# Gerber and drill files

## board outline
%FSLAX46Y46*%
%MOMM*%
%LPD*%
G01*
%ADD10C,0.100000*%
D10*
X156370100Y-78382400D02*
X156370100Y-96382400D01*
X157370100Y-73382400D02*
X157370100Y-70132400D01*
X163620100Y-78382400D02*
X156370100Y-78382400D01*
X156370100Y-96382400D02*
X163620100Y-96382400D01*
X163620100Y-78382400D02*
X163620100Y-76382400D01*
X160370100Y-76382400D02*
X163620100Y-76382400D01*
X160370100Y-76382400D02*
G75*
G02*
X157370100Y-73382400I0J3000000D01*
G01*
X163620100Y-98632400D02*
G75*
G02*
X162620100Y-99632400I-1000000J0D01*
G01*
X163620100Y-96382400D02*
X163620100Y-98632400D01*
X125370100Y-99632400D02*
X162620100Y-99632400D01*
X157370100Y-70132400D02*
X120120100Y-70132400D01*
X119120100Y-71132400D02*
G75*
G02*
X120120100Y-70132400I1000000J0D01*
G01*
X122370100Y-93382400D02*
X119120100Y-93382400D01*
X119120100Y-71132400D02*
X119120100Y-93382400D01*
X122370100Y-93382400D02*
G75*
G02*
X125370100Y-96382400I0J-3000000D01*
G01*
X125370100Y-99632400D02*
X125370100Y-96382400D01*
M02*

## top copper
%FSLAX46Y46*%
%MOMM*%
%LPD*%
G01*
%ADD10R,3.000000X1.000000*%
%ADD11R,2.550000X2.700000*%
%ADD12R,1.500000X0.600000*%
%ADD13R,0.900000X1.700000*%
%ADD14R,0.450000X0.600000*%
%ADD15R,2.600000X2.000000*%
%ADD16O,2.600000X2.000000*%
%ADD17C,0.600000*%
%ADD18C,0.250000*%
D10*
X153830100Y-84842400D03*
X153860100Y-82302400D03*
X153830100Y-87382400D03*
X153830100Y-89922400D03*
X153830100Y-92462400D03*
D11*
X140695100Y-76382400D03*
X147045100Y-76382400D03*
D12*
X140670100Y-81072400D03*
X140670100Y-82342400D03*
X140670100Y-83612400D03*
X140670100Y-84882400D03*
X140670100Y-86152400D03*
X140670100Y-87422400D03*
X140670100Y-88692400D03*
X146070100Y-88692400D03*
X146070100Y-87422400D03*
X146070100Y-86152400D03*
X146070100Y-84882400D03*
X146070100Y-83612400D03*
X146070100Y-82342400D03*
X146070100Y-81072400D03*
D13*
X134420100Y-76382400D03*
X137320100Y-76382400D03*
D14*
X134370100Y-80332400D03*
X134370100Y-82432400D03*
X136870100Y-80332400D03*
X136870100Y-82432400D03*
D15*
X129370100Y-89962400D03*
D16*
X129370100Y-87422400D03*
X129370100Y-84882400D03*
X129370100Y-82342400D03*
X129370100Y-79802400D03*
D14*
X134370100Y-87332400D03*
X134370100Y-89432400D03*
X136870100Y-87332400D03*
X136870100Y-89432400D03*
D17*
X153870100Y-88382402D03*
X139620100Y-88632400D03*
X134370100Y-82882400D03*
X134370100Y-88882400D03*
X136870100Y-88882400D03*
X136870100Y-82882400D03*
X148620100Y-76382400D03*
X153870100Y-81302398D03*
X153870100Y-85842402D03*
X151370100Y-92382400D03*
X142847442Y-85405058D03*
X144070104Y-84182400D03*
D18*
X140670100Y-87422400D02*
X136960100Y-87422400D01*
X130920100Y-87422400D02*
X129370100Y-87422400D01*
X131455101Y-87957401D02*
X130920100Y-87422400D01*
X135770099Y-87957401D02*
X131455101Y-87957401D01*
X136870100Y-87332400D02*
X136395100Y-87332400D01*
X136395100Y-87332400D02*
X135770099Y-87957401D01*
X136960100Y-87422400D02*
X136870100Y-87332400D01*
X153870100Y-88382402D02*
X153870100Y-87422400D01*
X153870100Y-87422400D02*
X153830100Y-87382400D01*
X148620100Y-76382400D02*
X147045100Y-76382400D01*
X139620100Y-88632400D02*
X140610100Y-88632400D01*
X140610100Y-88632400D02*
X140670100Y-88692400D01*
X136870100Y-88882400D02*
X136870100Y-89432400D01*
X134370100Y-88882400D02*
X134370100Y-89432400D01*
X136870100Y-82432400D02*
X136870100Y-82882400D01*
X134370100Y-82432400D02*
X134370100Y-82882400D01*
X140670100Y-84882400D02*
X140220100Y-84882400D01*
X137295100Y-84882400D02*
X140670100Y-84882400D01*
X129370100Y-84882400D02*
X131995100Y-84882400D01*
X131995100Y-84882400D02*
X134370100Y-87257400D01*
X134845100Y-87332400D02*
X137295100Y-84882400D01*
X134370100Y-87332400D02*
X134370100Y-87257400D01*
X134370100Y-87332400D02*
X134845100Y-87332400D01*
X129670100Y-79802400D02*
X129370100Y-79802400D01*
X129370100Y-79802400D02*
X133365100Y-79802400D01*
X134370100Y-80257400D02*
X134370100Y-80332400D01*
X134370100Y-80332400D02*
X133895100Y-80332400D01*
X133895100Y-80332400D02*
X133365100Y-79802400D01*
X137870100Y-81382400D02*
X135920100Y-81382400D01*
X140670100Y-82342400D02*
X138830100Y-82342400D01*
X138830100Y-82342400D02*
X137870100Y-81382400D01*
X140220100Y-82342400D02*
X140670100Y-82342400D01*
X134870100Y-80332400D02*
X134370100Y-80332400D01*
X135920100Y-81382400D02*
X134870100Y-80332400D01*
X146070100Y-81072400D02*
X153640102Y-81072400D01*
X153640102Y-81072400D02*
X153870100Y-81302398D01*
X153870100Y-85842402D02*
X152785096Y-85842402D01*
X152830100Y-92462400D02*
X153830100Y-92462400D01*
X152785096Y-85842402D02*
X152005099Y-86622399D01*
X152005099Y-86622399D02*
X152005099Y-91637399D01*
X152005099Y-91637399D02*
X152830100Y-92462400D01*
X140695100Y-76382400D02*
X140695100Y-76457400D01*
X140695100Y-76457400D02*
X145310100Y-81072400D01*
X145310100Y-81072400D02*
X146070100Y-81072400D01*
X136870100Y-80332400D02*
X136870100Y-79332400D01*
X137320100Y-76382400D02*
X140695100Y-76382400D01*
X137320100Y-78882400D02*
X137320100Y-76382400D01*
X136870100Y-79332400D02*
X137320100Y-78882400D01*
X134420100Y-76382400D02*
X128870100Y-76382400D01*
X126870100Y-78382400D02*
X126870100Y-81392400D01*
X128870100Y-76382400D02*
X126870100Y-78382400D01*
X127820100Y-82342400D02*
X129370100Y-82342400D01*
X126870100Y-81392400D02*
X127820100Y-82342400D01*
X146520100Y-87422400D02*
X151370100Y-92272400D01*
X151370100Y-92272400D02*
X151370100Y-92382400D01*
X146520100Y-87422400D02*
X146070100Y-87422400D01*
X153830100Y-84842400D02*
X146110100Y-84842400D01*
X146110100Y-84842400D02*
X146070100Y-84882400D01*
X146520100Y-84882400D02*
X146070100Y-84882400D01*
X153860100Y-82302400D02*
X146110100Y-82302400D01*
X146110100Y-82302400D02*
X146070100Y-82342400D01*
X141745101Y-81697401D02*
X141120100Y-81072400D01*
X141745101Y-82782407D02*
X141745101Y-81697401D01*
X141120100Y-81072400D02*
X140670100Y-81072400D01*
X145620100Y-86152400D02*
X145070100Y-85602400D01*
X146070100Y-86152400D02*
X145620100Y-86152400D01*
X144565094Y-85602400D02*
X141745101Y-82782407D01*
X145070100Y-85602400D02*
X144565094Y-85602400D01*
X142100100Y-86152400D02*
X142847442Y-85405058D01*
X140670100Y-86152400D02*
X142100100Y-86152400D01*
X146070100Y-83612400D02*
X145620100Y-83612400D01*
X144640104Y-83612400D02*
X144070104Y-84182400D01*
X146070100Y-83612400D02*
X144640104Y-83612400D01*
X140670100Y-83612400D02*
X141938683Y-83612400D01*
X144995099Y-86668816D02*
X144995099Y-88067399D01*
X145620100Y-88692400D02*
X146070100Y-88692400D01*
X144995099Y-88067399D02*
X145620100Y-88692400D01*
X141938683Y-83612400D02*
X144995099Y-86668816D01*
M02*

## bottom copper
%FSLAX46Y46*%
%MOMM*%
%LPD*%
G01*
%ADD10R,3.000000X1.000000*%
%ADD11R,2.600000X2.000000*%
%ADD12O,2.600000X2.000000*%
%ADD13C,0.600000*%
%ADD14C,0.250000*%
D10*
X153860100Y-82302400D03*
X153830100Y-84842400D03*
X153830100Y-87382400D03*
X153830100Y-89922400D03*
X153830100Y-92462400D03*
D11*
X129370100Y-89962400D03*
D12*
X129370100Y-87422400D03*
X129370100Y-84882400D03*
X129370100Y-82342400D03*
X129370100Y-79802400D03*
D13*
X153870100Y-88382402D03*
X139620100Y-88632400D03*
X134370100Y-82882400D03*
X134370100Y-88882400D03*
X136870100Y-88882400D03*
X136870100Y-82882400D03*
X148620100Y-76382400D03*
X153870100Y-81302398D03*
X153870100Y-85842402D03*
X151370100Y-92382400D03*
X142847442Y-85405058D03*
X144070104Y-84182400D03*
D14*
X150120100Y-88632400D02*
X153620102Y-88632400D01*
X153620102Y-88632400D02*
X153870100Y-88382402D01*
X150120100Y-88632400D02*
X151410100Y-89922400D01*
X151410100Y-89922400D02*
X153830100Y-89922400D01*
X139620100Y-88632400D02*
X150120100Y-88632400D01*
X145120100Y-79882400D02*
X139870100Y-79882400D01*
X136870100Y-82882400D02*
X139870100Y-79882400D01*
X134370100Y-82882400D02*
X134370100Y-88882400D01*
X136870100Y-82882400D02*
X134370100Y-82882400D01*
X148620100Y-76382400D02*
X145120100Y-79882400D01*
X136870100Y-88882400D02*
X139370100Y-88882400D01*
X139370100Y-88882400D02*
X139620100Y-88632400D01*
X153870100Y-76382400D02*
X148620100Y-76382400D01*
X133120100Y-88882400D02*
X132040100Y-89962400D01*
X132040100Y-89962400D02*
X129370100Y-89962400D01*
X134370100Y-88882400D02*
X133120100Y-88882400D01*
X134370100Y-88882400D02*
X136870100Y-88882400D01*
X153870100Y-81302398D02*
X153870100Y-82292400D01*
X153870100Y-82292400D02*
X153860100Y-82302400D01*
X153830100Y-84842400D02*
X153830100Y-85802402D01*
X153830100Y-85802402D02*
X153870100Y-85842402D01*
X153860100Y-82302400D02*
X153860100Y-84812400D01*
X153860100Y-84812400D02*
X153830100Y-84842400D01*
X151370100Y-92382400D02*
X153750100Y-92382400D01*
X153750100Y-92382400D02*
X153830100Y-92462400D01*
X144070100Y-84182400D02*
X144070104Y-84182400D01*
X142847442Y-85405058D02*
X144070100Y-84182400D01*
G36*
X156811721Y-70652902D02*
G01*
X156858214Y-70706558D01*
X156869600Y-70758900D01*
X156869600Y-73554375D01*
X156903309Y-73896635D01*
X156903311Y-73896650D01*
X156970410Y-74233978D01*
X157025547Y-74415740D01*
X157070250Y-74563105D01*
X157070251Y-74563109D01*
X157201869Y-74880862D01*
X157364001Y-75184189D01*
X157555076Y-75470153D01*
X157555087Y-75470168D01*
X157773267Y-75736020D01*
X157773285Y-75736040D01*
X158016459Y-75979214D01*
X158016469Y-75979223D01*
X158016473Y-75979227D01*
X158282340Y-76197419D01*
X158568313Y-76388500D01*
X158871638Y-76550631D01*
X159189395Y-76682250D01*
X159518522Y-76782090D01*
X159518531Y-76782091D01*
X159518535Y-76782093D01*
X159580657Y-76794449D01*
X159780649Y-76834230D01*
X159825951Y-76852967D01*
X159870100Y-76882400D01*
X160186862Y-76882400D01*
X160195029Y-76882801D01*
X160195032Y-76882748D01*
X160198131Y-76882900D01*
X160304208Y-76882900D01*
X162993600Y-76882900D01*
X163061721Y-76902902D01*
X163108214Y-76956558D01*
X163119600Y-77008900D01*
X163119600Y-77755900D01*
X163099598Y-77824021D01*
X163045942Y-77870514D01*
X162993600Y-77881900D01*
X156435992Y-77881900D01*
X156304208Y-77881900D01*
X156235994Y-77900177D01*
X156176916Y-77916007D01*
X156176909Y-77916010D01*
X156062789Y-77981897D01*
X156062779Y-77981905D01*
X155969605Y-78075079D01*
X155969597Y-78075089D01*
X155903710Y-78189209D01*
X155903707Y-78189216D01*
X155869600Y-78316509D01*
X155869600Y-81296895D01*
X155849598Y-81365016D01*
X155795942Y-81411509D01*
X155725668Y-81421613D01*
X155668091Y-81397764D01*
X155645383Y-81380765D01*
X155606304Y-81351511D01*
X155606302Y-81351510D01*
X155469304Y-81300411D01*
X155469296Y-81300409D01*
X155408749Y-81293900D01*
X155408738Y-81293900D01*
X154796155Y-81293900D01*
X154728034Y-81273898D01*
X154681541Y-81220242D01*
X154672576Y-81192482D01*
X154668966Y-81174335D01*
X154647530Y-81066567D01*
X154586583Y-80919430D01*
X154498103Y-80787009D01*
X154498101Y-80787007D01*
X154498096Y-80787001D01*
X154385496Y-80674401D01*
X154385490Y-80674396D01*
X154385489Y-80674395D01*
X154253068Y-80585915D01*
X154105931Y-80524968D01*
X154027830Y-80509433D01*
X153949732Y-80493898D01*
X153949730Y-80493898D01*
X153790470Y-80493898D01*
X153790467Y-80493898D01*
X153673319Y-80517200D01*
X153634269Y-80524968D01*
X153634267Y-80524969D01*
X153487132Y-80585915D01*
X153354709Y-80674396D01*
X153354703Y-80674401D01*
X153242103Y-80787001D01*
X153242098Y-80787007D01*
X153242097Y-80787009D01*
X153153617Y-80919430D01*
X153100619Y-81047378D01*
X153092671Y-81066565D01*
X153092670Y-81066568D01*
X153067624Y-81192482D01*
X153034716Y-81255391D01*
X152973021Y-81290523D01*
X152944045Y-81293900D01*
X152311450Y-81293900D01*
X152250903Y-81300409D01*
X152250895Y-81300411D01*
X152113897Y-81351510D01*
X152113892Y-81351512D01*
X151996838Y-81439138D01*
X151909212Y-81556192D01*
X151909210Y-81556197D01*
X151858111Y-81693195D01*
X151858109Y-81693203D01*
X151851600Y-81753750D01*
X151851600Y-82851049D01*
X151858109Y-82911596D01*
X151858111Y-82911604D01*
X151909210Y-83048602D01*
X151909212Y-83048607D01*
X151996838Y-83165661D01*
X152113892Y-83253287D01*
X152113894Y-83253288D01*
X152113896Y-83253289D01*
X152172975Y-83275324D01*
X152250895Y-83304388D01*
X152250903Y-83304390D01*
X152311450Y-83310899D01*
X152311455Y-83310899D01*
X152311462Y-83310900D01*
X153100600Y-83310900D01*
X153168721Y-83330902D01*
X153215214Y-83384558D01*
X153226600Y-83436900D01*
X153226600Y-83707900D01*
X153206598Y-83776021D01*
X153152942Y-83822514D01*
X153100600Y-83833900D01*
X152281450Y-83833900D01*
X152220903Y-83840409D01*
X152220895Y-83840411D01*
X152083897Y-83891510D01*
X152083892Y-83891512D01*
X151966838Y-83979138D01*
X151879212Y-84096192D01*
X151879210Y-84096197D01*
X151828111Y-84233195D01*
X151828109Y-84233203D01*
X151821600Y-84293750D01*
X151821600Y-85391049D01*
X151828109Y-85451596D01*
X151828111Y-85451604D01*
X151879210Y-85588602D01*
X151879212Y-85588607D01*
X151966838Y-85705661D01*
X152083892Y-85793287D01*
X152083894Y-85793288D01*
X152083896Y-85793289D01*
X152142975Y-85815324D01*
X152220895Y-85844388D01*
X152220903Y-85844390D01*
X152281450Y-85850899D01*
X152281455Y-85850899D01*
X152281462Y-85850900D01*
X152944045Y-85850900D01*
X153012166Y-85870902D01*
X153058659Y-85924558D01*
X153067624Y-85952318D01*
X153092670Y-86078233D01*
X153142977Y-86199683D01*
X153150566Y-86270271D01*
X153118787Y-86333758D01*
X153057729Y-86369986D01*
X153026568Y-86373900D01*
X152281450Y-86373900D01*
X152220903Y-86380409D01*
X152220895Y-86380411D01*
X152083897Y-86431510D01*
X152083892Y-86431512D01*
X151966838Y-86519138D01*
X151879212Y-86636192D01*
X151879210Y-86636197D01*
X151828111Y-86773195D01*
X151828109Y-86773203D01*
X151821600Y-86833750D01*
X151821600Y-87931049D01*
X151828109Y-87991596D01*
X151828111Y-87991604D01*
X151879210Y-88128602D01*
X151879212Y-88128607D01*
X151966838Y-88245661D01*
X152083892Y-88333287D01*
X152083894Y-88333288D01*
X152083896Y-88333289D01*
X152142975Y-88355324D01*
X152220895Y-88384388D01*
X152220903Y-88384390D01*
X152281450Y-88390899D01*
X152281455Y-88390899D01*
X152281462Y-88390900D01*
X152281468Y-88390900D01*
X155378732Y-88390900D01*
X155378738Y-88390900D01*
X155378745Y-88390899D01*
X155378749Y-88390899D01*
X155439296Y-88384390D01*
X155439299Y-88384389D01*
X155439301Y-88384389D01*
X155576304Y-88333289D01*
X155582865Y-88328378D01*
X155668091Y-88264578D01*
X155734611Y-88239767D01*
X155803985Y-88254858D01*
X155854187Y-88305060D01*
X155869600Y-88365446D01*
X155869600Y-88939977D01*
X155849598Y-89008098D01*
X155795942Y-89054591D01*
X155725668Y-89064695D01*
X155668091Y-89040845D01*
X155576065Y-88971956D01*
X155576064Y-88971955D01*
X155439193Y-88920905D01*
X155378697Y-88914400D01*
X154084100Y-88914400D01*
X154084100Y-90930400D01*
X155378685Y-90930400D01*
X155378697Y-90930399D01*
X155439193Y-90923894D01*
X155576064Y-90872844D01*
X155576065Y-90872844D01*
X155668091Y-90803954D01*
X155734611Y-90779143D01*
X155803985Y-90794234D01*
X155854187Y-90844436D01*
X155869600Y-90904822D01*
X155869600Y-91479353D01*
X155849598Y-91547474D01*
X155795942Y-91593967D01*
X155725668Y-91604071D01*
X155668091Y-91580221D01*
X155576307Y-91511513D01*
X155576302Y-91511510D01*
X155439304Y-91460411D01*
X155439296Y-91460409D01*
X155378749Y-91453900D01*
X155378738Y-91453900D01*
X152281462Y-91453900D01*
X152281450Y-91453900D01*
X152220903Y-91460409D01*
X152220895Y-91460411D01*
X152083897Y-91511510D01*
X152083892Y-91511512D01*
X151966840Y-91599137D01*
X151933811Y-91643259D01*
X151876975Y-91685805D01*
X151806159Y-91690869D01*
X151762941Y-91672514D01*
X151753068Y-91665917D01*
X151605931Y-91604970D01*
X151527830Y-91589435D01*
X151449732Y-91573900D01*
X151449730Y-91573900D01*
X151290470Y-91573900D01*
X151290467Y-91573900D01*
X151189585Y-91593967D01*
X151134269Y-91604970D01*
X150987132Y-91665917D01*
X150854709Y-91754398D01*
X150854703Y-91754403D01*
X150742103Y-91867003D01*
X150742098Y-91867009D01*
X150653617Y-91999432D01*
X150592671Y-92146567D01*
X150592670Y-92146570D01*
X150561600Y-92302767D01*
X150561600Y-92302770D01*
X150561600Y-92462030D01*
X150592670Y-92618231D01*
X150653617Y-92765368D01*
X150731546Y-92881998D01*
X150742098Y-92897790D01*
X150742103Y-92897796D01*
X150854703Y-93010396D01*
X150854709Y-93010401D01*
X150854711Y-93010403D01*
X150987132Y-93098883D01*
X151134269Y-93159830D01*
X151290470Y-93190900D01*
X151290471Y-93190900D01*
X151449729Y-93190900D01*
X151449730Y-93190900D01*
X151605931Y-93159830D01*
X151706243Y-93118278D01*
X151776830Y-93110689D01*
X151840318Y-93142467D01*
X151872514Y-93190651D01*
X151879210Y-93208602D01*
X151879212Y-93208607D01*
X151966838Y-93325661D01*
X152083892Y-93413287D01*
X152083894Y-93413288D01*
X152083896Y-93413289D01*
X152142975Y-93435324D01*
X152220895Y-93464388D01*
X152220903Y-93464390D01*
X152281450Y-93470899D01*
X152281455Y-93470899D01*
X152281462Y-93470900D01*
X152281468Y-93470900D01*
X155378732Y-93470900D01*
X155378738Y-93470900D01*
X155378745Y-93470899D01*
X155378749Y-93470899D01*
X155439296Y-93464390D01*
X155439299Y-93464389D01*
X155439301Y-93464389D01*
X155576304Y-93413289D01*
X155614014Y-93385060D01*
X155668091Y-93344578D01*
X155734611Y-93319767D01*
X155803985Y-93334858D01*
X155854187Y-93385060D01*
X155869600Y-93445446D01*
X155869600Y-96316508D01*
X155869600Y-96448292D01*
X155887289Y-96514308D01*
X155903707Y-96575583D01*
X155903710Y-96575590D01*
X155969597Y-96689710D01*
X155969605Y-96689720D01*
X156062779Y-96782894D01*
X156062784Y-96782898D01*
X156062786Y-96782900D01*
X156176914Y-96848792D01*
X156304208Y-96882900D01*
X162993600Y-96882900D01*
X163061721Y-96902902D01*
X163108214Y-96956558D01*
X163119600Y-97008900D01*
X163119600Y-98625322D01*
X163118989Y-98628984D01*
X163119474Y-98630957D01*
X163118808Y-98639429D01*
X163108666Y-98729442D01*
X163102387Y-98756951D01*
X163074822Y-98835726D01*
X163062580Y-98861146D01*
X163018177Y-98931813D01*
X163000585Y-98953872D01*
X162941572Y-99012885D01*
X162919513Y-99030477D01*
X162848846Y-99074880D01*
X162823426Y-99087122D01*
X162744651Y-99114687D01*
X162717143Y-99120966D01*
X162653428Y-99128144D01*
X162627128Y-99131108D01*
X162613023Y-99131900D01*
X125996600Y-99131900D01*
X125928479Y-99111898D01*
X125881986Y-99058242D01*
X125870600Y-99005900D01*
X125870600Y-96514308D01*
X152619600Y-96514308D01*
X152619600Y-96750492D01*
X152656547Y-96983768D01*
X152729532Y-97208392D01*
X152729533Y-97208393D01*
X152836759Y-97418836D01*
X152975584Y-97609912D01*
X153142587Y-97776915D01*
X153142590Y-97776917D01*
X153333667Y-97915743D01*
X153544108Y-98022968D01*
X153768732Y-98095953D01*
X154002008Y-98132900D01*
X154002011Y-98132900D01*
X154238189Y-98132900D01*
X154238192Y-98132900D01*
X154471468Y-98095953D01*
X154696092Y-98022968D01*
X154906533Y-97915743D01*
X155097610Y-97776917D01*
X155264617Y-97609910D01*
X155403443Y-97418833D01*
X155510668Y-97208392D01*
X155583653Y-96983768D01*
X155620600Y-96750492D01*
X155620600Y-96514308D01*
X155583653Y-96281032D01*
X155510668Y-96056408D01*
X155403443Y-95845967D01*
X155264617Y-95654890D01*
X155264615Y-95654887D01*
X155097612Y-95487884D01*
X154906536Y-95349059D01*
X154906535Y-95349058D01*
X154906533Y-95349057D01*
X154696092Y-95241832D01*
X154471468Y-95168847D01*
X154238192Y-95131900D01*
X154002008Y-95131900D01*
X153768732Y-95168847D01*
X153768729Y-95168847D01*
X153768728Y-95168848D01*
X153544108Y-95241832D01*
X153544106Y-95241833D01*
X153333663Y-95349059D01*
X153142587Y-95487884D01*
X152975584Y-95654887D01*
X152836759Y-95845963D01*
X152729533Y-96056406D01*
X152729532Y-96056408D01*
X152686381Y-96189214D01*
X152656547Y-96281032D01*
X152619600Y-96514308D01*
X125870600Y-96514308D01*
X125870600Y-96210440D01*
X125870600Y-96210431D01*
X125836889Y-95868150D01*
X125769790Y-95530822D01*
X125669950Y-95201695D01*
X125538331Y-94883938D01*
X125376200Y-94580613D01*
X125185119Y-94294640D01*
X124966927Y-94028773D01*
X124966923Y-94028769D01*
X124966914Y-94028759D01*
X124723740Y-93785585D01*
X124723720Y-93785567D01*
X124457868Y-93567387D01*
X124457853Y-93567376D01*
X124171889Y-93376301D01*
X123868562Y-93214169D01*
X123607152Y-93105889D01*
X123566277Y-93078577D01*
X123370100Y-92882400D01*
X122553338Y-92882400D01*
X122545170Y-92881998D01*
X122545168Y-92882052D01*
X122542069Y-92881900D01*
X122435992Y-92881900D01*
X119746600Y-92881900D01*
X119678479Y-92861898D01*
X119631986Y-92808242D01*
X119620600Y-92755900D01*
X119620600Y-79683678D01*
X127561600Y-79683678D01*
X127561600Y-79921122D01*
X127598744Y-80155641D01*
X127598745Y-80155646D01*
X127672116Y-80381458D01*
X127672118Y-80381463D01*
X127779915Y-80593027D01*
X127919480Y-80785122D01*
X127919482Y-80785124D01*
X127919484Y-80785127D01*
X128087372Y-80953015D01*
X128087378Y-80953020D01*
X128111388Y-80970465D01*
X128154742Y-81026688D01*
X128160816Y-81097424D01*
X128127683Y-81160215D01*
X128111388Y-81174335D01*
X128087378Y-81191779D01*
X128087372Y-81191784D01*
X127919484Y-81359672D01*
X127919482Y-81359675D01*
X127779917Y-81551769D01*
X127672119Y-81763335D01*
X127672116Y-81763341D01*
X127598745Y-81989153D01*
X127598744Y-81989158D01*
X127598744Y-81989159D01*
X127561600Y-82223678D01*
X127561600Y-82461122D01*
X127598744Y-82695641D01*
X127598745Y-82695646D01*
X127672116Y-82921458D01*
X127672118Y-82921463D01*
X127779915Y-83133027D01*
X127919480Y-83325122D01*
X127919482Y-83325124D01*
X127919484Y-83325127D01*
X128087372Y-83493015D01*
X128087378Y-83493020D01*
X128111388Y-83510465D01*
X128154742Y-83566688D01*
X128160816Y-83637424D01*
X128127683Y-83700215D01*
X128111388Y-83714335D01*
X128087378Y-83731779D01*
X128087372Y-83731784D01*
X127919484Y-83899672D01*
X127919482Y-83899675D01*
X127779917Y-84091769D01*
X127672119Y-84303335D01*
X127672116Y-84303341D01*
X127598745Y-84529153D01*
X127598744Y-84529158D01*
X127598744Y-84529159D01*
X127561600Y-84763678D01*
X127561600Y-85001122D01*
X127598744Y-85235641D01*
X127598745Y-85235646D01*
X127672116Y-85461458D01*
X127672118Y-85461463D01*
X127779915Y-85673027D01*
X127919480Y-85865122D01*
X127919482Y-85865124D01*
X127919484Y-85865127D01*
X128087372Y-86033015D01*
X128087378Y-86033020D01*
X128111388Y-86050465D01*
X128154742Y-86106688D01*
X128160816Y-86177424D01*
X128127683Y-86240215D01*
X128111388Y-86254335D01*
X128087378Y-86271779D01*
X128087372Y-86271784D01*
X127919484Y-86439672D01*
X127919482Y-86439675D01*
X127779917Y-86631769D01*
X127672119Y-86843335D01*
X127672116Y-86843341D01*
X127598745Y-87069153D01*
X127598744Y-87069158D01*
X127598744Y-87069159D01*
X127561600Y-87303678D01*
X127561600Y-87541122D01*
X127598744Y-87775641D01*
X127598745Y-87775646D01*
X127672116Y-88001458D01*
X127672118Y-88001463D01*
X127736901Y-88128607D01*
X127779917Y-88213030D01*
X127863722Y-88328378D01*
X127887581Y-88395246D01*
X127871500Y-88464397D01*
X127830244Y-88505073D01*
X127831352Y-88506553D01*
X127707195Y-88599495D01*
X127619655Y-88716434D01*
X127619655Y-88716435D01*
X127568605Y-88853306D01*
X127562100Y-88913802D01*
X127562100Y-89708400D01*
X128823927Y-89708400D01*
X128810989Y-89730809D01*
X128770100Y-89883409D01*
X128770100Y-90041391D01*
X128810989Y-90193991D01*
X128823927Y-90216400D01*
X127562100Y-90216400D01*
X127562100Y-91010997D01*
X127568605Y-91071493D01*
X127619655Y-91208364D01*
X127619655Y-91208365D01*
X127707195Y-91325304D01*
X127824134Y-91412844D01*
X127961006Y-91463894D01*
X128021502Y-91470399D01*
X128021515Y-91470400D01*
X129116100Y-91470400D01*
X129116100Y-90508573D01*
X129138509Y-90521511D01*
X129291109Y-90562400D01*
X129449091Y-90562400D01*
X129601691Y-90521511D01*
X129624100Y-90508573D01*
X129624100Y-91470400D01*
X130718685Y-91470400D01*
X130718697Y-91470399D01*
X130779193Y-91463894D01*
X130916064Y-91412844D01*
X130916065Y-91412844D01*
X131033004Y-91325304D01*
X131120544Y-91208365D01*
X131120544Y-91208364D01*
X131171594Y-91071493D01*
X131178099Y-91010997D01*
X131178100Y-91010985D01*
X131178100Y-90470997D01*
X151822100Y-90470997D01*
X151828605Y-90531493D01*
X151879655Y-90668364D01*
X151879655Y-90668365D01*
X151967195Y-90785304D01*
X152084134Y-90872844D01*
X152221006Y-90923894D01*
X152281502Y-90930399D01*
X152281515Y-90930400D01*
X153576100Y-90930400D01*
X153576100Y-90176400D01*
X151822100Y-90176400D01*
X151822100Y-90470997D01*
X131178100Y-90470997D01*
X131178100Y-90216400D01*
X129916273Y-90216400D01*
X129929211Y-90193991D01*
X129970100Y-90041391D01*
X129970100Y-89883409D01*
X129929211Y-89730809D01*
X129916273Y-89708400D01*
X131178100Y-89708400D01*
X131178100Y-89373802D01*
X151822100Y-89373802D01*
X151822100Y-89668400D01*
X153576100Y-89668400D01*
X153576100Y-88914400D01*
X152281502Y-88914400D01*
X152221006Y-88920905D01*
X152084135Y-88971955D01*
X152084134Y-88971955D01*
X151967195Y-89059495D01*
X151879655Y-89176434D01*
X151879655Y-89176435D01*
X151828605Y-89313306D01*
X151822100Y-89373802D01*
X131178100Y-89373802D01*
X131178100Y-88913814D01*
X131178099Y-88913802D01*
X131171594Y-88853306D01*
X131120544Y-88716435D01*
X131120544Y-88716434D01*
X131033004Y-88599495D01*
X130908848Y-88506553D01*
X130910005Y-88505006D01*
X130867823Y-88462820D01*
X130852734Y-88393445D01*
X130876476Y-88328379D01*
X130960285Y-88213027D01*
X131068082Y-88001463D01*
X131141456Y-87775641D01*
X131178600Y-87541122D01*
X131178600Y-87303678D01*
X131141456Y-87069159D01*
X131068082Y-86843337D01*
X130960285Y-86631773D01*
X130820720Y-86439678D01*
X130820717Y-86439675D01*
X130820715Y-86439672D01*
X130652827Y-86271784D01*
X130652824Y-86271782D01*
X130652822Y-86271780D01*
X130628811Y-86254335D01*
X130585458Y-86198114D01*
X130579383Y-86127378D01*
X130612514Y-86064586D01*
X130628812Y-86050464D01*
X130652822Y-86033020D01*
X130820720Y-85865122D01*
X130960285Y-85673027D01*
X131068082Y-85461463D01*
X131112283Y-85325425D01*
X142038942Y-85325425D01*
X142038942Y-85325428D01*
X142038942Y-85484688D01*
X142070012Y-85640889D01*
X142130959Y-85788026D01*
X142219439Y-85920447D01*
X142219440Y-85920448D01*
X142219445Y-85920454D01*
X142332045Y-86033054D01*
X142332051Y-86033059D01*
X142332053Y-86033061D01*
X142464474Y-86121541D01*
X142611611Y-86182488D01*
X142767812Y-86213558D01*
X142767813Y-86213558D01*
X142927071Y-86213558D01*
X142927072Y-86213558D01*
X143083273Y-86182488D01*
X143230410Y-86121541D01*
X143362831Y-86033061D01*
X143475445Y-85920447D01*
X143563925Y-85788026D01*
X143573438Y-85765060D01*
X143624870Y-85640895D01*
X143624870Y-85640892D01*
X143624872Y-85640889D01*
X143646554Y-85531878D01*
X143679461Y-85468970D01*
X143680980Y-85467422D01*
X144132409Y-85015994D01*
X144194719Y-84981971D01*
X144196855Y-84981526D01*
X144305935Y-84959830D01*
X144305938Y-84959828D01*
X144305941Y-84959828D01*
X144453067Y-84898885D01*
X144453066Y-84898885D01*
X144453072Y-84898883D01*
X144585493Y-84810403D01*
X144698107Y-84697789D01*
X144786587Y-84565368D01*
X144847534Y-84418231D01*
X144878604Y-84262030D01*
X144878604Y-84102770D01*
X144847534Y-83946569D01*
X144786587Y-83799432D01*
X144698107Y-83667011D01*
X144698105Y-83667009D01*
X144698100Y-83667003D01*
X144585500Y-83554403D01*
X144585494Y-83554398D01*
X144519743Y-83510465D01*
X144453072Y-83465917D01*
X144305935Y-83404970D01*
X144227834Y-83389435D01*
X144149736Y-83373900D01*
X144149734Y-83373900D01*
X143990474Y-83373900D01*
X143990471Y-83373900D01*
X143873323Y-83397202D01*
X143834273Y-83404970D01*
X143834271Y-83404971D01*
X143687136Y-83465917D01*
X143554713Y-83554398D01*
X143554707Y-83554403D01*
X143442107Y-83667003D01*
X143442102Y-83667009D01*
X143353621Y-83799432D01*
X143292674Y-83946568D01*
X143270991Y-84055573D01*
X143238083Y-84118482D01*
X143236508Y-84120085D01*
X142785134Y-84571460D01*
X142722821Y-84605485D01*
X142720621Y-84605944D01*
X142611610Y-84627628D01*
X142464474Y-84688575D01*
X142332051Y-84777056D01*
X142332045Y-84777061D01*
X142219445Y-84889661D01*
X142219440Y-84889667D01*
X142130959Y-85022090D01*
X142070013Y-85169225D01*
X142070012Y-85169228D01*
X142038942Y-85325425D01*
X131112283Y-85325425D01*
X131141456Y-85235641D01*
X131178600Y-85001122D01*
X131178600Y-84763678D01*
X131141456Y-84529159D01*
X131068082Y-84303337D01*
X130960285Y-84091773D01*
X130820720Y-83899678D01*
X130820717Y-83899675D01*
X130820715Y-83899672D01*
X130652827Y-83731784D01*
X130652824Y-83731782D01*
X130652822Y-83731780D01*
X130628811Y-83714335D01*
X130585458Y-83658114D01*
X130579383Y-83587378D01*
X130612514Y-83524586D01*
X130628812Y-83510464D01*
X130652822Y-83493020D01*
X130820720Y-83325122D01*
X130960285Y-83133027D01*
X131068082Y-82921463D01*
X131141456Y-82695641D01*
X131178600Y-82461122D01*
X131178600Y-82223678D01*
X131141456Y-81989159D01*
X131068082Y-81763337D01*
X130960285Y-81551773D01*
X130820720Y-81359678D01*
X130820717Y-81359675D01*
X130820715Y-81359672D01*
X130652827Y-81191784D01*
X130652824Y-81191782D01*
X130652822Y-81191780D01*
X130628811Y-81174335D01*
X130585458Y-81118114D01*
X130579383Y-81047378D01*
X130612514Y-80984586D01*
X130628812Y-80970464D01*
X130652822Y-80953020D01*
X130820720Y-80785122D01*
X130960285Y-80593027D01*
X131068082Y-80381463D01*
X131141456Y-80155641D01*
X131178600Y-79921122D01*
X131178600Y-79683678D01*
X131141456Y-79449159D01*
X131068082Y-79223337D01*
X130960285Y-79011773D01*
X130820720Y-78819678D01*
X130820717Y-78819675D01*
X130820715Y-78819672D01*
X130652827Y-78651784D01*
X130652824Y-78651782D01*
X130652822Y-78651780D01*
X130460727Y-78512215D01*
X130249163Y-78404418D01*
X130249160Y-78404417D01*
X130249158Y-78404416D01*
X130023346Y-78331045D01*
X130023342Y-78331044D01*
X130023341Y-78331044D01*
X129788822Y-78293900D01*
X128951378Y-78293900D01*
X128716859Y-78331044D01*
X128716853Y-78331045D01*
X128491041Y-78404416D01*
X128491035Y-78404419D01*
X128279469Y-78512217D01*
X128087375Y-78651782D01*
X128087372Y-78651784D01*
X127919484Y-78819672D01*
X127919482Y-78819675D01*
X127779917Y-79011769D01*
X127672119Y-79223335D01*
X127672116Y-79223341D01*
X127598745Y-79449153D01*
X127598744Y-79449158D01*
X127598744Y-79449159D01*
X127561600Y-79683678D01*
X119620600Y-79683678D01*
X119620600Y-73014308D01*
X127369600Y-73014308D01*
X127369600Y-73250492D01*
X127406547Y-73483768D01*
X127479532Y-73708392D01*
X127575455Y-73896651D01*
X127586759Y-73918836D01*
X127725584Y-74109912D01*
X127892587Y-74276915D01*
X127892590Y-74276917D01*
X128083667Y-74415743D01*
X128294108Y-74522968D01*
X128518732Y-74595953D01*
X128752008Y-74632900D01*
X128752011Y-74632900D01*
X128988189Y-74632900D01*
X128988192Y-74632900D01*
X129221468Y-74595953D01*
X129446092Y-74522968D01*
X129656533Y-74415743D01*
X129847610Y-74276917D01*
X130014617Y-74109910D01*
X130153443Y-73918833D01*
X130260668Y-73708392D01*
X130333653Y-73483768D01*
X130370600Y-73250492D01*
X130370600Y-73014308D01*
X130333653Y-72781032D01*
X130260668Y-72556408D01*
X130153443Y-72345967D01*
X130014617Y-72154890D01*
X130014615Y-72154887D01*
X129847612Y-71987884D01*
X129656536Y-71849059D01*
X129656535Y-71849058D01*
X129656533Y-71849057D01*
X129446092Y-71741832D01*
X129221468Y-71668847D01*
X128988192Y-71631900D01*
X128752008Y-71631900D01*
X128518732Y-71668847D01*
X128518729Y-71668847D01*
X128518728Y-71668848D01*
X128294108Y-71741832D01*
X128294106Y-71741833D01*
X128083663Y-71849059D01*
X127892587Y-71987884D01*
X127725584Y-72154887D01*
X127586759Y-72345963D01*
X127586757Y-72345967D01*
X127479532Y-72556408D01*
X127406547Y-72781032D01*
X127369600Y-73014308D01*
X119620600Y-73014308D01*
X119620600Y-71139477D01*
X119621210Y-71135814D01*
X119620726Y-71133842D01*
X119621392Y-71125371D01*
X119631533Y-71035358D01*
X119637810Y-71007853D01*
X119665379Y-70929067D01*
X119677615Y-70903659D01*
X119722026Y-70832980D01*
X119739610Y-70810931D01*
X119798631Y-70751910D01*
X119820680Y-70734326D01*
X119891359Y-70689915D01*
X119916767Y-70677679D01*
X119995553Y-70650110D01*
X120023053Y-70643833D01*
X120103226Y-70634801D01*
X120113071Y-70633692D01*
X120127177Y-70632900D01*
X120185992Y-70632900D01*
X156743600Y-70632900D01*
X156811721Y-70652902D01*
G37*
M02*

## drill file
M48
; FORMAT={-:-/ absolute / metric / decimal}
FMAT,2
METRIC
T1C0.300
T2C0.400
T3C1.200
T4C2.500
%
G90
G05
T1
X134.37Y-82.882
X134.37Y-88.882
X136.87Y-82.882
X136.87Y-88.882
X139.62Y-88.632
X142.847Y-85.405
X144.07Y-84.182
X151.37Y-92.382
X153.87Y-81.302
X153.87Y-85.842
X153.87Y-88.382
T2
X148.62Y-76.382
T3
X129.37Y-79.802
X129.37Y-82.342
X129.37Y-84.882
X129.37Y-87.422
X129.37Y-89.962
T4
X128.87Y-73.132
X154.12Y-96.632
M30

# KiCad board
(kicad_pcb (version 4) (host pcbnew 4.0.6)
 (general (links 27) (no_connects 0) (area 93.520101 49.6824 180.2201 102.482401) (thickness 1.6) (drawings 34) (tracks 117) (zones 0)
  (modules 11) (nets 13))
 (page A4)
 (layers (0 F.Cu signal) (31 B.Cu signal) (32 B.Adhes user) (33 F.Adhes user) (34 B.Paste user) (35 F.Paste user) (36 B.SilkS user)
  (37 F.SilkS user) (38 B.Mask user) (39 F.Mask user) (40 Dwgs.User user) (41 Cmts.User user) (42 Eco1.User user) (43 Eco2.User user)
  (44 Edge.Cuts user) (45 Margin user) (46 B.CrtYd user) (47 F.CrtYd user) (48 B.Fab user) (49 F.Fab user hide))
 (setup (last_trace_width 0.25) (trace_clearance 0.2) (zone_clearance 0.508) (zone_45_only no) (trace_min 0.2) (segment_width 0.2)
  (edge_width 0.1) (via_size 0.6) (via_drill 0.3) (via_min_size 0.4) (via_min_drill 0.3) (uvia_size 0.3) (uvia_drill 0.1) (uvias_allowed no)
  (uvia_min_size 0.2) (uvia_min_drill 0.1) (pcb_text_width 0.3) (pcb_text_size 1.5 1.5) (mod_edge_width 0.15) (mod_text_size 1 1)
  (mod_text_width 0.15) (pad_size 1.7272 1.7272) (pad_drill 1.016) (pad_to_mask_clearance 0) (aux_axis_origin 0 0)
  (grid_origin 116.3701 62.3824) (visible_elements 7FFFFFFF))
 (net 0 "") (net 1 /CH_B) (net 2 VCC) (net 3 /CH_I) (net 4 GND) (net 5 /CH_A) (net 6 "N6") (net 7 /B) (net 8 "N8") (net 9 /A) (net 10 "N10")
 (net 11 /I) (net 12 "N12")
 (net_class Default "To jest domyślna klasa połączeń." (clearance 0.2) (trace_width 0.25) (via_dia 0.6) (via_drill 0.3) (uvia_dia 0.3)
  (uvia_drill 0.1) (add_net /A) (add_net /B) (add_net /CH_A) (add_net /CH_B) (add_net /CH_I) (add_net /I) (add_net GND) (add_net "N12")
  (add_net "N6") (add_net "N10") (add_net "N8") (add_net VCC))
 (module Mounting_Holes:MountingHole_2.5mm (layer F.Cu) (at 154.1201 96.6324)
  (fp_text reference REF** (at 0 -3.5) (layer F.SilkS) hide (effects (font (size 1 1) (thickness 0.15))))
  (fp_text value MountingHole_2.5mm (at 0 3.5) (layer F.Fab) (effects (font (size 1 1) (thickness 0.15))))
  (pad 1 np_thru_hole circle (at 0 0) (size 2.5 2.5) (drill 2.5) (layers *.Cu *.Mask)))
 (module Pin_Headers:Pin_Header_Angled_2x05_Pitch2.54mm (layer F.Cu) (at 153.8301 82.3024)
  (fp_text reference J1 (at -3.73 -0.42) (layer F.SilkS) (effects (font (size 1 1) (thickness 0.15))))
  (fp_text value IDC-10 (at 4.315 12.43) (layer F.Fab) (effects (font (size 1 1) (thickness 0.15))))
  (pad 8 smd rect (at 0 2.54) (size 3 1) (layers F.Cu F.Paste F.Mask) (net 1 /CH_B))
  (pad 9 smd rect (at 0.03 0) (size 3 1) (layers B.Cu B.Adhes B.Mask) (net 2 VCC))
  (pad 10 smd rect (at 0.03 0) (size 3 1) (layers F.Cu F.Paste F.Mask) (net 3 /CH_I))
  (pad 6 smd rect (at 0 5.08) (size 3 1) (layers F.Cu F.Paste F.Mask) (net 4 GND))
  (pad 4 smd rect (at 0 7.62) (size 3 1) (layers F.Cu F.Paste F.Mask))
  (pad 2 smd rect (at 0 10.16) (size 3 1) (layers F.Cu F.Paste F.Mask) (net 2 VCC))
  (pad 7 smd rect (at 0 2.54) (size 3 1) (layers B.Cu B.Adhes B.Mask) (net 2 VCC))
  (pad 5 smd rect (at 0 5.08) (size 3 1) (layers B.Cu B.Adhes B.Mask))
  (pad 3 smd rect (at 0 7.62) (size 3 1) (layers B.Cu B.Adhes B.Mask) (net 4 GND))
  (pad 1 smd rect (at 0 10.16) (size 3 1) (layers B.Cu B.Adhes B.Mask) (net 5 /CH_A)))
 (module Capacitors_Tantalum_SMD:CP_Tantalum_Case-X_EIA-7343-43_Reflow (layer F.Cu) (at 143.8701 76.3824)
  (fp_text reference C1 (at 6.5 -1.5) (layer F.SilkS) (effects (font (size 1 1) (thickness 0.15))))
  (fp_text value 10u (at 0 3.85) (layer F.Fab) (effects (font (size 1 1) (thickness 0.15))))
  (pad 1 smd rect (at -3.175 0) (size 2.55 2.7) (layers F.Cu F.Paste F.Mask) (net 2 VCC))
  (pad 2 smd rect (at 3.175 0) (size 2.55 2.7) (layers F.Cu F.Paste F.Mask) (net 4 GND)))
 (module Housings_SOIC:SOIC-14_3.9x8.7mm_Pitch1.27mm (layer F.Cu) (at 143.3701 84.8824)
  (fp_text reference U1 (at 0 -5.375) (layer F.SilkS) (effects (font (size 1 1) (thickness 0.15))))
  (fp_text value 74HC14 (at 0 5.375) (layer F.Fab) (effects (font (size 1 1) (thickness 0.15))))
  (pad 1 smd rect (at -2.7 -3.81) (size 1.5 0.6) (layers F.Cu F.Paste F.Mask) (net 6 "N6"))
  (pad 2 smd rect (at -2.7 -2.54) (size 1.5 0.6) (layers F.Cu F.Paste F.Mask) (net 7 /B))
  (pad 3 smd rect (at -2.7 -1.27) (size 1.5 0.6) (layers F.Cu F.Paste F.Mask) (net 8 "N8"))
  (pad 4 smd rect (at -2.7 0) (size 1.5 0.6) (layers F.Cu F.Paste F.Mask) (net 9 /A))
  (pad 5 smd rect (at -2.7 1.27) (size 1.5 0.6) (layers F.Cu F.Paste F.Mask) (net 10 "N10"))
  (pad 6 smd rect (at -2.7 2.54) (size 1.5 0.6) (layers F.Cu F.Paste F.Mask) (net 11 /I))
  (pad 7 smd rect (at -2.7 3.81) (size 1.5 0.6) (layers F.Cu F.Paste F.Mask) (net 4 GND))
  (pad 8 smd rect (at 2.7 3.81) (size 1.5 0.6) (layers F.Cu F.Paste F.Mask) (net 8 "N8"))
  (pad 9 smd rect (at 2.7 2.54) (size 1.5 0.6) (layers F.Cu F.Paste F.Mask) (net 5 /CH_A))
  (pad 10 smd rect (at 2.7 1.27) (size 1.5 0.6) (layers F.Cu F.Paste F.Mask) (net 6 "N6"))
  (pad 11 smd rect (at 2.7 0) (size 1.5 0.6) (layers F.Cu F.Paste F.Mask) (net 1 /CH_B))
  (pad 12 smd rect (at 2.7 -1.27) (size 1.5 0.6) (layers F.Cu F.Paste F.Mask) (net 10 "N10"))
  (pad 13 smd rect (at 2.7 -2.54) (size 1.5 0.6) (layers F.Cu F.Paste F.Mask) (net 3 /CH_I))
  (pad 14 smd rect (at 2.7 -3.81) (size 1.5 0.6) (layers F.Cu F.Paste F.Mask) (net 2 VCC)))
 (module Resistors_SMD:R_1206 (layer F.Cu) (at 135.8701 76.3824)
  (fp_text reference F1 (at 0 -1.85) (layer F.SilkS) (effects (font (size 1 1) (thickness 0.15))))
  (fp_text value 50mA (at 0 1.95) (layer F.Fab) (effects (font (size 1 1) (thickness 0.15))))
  (pad 1 smd rect (at -1.45 0) (size 0.9 1.7) (layers F.Cu F.Paste F.Mask) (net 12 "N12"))
  (pad 2 smd rect (at 1.45 0) (size 0.9 1.7) (layers F.Cu F.Paste F.Mask) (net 2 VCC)))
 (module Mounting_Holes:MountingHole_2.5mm (layer F.Cu) (at 128.8701 73.1324)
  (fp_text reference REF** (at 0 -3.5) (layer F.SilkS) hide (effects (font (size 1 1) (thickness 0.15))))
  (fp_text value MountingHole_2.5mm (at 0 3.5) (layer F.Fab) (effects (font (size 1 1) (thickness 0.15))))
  (pad 1 np_thru_hole circle (at 0 0) (size 2.5 2.5) (drill 2.5) (layers *.Cu *.Mask)))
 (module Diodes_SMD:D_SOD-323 (layer F.Cu) (at 134.3701 81.3824 270)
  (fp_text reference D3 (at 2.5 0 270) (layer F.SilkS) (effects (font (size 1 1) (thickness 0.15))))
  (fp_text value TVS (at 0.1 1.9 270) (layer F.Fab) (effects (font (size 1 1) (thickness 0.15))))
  (pad 1 smd rect (at -1.05 0 270) (size 0.6 0.45) (layers F.Cu F.Paste F.Mask) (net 7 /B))
  (pad 2 smd rect (at 1.05 0 270) (size 0.6 0.45) (layers F.Cu F.Paste F.Mask) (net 4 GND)))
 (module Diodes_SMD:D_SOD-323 (layer F.Cu) (at 136.8701 81.3824 270)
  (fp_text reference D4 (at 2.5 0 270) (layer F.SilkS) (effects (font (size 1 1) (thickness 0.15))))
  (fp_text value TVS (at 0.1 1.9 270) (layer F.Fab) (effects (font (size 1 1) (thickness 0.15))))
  (pad 1 smd rect (at -1.05 0 270) (size 0.6 0.45) (layers F.Cu F.Paste F.Mask) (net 2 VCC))
  (pad 2 smd rect (at 1.05 0 270) (size 0.6 0.45) (layers F.Cu F.Paste F.Mask) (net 4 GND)))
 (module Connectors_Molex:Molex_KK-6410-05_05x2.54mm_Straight (layer F.Cu) (at 129.3701 89.9624 90)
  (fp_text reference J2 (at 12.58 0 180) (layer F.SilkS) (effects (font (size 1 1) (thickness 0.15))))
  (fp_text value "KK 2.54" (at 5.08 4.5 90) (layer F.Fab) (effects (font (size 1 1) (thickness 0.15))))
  (pad 1 thru_hole rect (at 0 0 90) (size 2 2.6) (drill 1.2) (layers *.Cu *.Mask) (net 4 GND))
  (pad 2 thru_hole oval (at 2.54 0 90) (size 2 2.6) (drill 1.2) (layers *.Cu *.Mask) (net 11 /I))
  (pad 3 thru_hole oval (at 5.08 0 90) (size 2 2.6) (drill 1.2) (layers *.Cu *.Mask) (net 9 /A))
  (pad 4 thru_hole oval (at 7.62 0 90) (size 2 2.6) (drill 1.2) (layers *.Cu *.Mask) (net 12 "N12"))
  (pad 5 thru_hole oval (at 10.16 0 90) (size 2 2.6) (drill 1.2) (layers *.Cu *.Mask) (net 7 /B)))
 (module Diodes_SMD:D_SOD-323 (layer F.Cu) (at 134.3701 88.3824 270)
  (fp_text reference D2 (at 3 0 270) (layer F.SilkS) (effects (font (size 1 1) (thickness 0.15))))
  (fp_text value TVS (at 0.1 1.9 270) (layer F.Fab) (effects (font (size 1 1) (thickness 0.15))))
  (pad 1 smd rect (at -1.05 0 270) (size 0.6 0.45) (layers F.Cu F.Paste F.Mask) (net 9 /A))
  (pad 2 smd rect (at 1.05 0 270) (size 0.6 0.45) (layers F.Cu F.Paste F.Mask) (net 4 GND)))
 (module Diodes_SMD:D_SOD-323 (layer F.Cu) (at 136.8701 88.3824 270)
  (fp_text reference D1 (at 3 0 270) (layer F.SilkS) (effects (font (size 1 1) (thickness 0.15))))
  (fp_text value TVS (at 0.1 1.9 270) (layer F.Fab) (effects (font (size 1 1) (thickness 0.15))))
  (pad 1 smd rect (at -1.05 0 270) (size 0.6 0.45) (layers F.Cu F.Paste F.Mask) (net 11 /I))
  (pad 2 smd rect (at 1.05 0 270) (size 0.6 0.45) (layers F.Cu F.Paste F.Mask) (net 4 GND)))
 (gr_line (start 156.3701 78.3824) (end 156.3701 96.3824) (layer Edge.Cuts) (width 0.1))
 (gr_line (start 157.3701 73.3824) (end 157.3701 70.1324) (layer Edge.Cuts) (width 0.1))
 (gr_line (start 163.6201 78.3824) (end 156.3701 78.3824) (layer Edge.Cuts) (width 0.1))
 (gr_line (start 156.3701 96.3824) (end 163.6201 96.3824) (layer Edge.Cuts) (width 0.1))
 (gr_line (start 163.6201 78.3824) (end 163.6201 76.3824) (layer Edge.Cuts) (width 0.1))
 (gr_line (start 160.3701 76.3824) (end 163.6201 76.3824) (layer Edge.Cuts) (width 0.1))
 (gr_arc (start 160.3701 73.3824) (end 160.3701 76.3824) (angle 90) (layer Edge.Cuts) (width 0.1))
 (gr_arc (start 162.6201 98.6324) (end 163.6201 98.6324) (angle 90) (layer Edge.Cuts) (width 0.1))
 (gr_line (start 163.6201 96.3824) (end 163.6201 98.6324) (layer Edge.Cuts) (width 0.1))
 (gr_line (start 125.3701 99.6324) (end 162.6201 99.6324) (layer Edge.Cuts) (width 0.1))
 (gr_line (start 157.3701 70.1324) (end 120.1201 70.1324) (layer Edge.Cuts) (width 0.1))
 (gr_arc (start 120.1201 71.1324) (end 119.1201 71.1324) (angle 90) (layer Edge.Cuts) (width 0.1))
 (gr_line (start 122.3701 93.3824) (end 119.1201 93.3824) (layer Edge.Cuts) (width 0.1))
 (gr_line (start 119.1201 71.1324) (end 119.1201 93.3824) (layer Edge.Cuts) (width 0.1))
 (gr_arc (start 122.3701 96.3824) (end 122.3701 93.3824) (angle 90) (layer Edge.Cuts) (width 0.1))
 (gr_line (start 125.3701 99.6324) (end 125.3701 96.3824) (layer Edge.Cuts) (width 0.1))
 (segment (start 140.6701 87.4224) (end 136.9601 87.4224) (width 0.25) (layer F.Cu) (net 11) (status 30))
 (segment (start 130.9201 87.4224) (end 129.3701 87.4224) (width 0.25) (layer F.Cu) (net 11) (status 20))
 (segment (start 131.455101 87.957401) (end 130.9201 87.4224) (width 0.25) (layer F.Cu) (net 11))
 (segment (start 135.770099 87.957401) (end 131.455101 87.957401) (width 0.25) (layer F.Cu) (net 11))
 (segment (start 136.8701 87.3324) (end 136.3951 87.3324) (width 0.25) (layer F.Cu) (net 11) (status 10))
 (segment (start 136.3951 87.3324) (end 135.770099 87.957401) (width 0.25) (layer F.Cu) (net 11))
 (segment (start 136.9601 87.4224) (end 136.8701 87.3324) (width 0.25) (layer F.Cu) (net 11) (status 30))
 (segment (start 153.8701 88.382402) (end 153.8701 87.4224) (width 0.25) (layer F.Cu) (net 4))
 (segment (start 153.8701 87.4224) (end 153.8301 87.3824) (width 0.25) (layer F.Cu) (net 4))
 (segment (start 150.1201 88.6324) (end 153.620102 88.6324) (width 0.25) (layer B.Cu) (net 4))
 (segment (start 153.620102 88.6324) (end 153.8701 88.382402) (width 0.25) (layer B.Cu) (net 4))
 (via (at 153.8701 88.382402) (size 0.6) (drill 0.3) (layers F.Cu B.Cu) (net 4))
 (segment (start 150.1201 88.6324) (end 151.4101 89.9224) (width 0.25) (layer B.Cu) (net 4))
 (segment (start 151.4101 89.9224) (end 153.8301 89.9224) (width 0.25) (layer B.Cu) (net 4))
 (segment (start 139.6201 88.6324) (end 150.1201 88.6324) (width 0.25) (layer B.Cu) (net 4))
 (segment (start 148.6201 76.3824) (end 147.0451 76.3824) (width 0.25) (layer F.Cu) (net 4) (status 20))
 (segment (start 139.6201 88.6324) (end 140.6101 88.6324) (width 0.25) (layer F.Cu) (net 4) (status 20))
 (segment (start 140.6101 88.6324) (end 140.6701 88.6924) (width 0.25) (layer F.Cu) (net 4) (status 30))
 (segment (start 136.8701 88.8824) (end 136.8701 89.4324) (width 0.25) (layer F.Cu) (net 4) (status 20))
 (segment (start 134.3701 88.8824) (end 134.3701 89.4324) (width 0.25) (layer F.Cu) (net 4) (status 20))
 (segment (start 136.8701 82.4324) (end 136.8701 82.8824) (width 0.25) (layer F.Cu) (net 4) (status 10))
 (segment (start 134.3701 82.4324) (end 134.3701 82.8824) (width 0.25) (layer F.Cu) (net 4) (status 10))
 (via (at 139.6201 88.6324) (size 0.6) (drill 0.3) (layers F.Cu B.Cu) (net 4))
 (via (at 134.3701 82.8824) (size 0.6) (drill 0.3) (layers F.Cu B.Cu) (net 4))
 (via (at 134.3701 88.8824) (size 0.6) (drill 0.3) (layers F.Cu B.Cu) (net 4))
 (via (at 136.8701 88.8824) (size 0.6) (drill 0.3) (layers F.Cu B.Cu) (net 4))
 (via (at 136.8701 82.8824) (size 0.6) (drill 0.3) (layers F.Cu B.Cu) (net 4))
 (via (at 148.6201 76.3824) (size 0.6) (drill 0.4) (layers F.Cu B.Cu) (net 4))
 (segment (start 145.1201 79.8824) (end 139.8701 79.8824) (width 0.25) (layer B.Cu) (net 4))
 (segment (start 136.8701 82.8824) (end 139.8701 79.8824) (width 0.25) (layer B.Cu) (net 4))
 (segment (start 134.3701 82.8824) (end 134.3701 88.8824) (width 0.25) (layer B.Cu) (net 4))
 (segment (start 136.8701 82.8824) (end 134.3701 82.8824) (width 0.25) (layer B.Cu) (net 4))
 (segment (start 148.6201 76.3824) (end 145.1201 79.8824) (width 0.25) (layer B.Cu) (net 4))
 (segment (start 136.8701 88.8824) (end 139.3701 88.8824) (width 0.25) (layer B.Cu) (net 4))
 (segment (start 139.3701 88.8824) (end 139.6201 88.6324) (width 0.25) (layer B.Cu) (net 4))
 (segment (start 153.8701 76.3824) (end 148.6201 76.3824) (width 0.25) (layer B.Cu) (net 4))
 (segment (start 133.1201 88.8824) (end 132.0401 89.9624) (width 0.25) (layer B.Cu) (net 4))
 (segment (start 132.0401 89.9624) (end 129.3701 89.9624) (width 0.25) (layer B.Cu) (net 4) (status 20))
 (segment (start 134.3701 88.8824) (end 133.1201 88.8824) (width 0.25) (layer B.Cu) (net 4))
 (segment (start 134.3701 88.8824) (end 136.8701 88.8824) (width 0.25) (layer B.Cu) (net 4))
 (segment (start 140.6701 84.8824) (end 140.2201 84.8824) (width 0.25) (layer F.Cu) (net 9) (status 30))
 (segment (start 137.2951 84.8824) (end 140.6701 84.8824) (width 0.25) (layer F.Cu) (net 9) (status 20))
 (segment (start 129.3701 84.8824) (end 131.9951 84.8824) (width 0.25) (layer F.Cu) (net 9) (status 10))
 (segment (start 131.9951 84.8824) (end 134.3701 87.2574) (width 0.25) (layer F.Cu) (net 9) (status 20))
 (segment (start 134.8451 87.3324) (end 137.2951 84.8824) (width 0.25) (layer F.Cu) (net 9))
 (segment (start 134.3701 87.3324) (end 134.3701 87.2574) (width 0.25) (layer F.Cu) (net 9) (status 30))
 (segment (start 134.3701 87.3324) (end 134.8451 87.3324) (width 0.25) (layer F.Cu) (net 9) (status 10))
 (segment (start 129.6701 79.8024) (end 129.3701 79.8024) (width 0.25) (layer F.Cu) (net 7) (status 30))
 (segment (start 129.3701 79.8024) (end 133.3651 79.8024) (width 0.25) (layer F.Cu) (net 7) (status 10))
 (segment (start 134.3701 80.2574) (end 134.3701 80.3324) (width 0.25) (layer F.Cu) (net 7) (status 30))
 (segment (start 134.3701 80.3324) (end 133.8951 80.3324) (width 0.25) (layer F.Cu) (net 7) (status 10))
 (segment (start 133.8951 80.3324) (end 133.3651 79.8024) (width 0.25) (layer F.Cu) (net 7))
 (segment (start 137.8701 81.3824) (end 135.9201 81.3824) (width 0.25) (layer F.Cu) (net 7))
 (segment (start 140.6701 82.3424) (end 138.8301 82.3424) (width 0.25) (layer F.Cu) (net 7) (status 10))
 (segment (start 138.8301 82.3424) (end 137.8701 81.3824) (width 0.25) (layer F.Cu) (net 7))
 (segment (start 140.2201 82.3424) (end 140.6701 82.3424) (width 0.25) (layer F.Cu) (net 7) (status 30))
 (segment (start 134.8701 80.3324) (end 134.3701 80.3324) (width 0.25) (layer F.Cu) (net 7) (status 20))
 (segment (start 135.9201 81.3824) (end 134.8701 80.3324) (width 0.25) (layer F.Cu) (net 7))
 (segment (start 153.8701 81.302398) (end 153.8701 82.2924) (width 0.25) (layer B.Cu) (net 2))
 (segment (start 153.8701 82.2924) (end 153.8601 82.3024) (width 0.25) (layer B.Cu) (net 2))
 (segment (start 146.0701 81.0724) (end 153.640102 81.0724) (width 0.25) (layer F.Cu) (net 2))
 (segment (start 153.640102 81.0724) (end 153.8701 81.302398) (width 0.25) (layer F.Cu) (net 2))
 (via (at 153.8701 81.302398) (size 0.6) (drill 0.3) (layers F.Cu B.Cu) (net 2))
 (segment (start 153.8701 85.842402) (end 152.785096 85.842402) (width 0.25) (layer F.Cu) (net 2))
 (segment (start 152.8301 92.4624) (end 153.8301 92.4624) (width 0.25) (layer F.Cu) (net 2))
 (segment (start 152.785096 85.842402) (end 152.005099 86.622399) (width 0.25) (layer F.Cu) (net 2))
 (segment (start 152.005099 86.622399) (end 152.005099 91.637399) (width 0.25) (layer F.Cu) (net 2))
 (segment (start 152.005099 91.637399) (end 152.8301 92.4624) (width 0.25) (layer F.Cu) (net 2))
 (segment (start 153.8301 84.8424) (end 153.8301 85.802402) (width 0.25) (layer B.Cu) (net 2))
 (segment (start 153.8301 85.802402) (end 153.8701 85.842402) (width 0.25) (layer B.Cu) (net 2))
 (via (at 153.8701 85.842402) (size 0.6) (drill 0.3) (layers F.Cu B.Cu) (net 2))
 (segment (start 153.8601 82.3024) (end 153.8601 84.8124) (width 0.25) (layer B.Cu) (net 2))
 (segment (start 153.8601 84.8124) (end 153.8301 84.8424) (width 0.25) (layer B.Cu) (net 2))
 (segment (start 140.6951 76.3824) (end 140.6951 76.4574) (width 0.25) (layer F.Cu) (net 2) (status 30))
 (segment (start 140.6951 76.4574) (end 145.3101 81.0724) (width 0.25) (layer F.Cu) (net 2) (status 10))
 (segment (start 145.3101 81.0724) (end 146.0701 81.0724) (width 0.25) (layer F.Cu) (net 2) (status 20))
 (segment (start 136.8701 80.3324) (end 136.8701 79.3324) (width 0.25) (layer F.Cu) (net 2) (status 10))
 (segment (start 137.3201 76.3824) (end 140.6951 76.3824) (width 0.25) (layer F.Cu) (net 2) (status 30))
 (segment (start 137.3201 78.8824) (end 137.3201 76.3824) (width 0.25) (layer F.Cu) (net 2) (status 20))
 (segment (start 136.8701 79.3324) (end 137.3201 78.8824) (width 0.25) (layer F.Cu) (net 2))
 (segment (start 134.4201 76.3824) (end 128.8701 76.3824) (width 0.25) (layer F.Cu) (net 12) (status 10))
 (segment (start 126.8701 78.3824) (end 126.8701 81.3924) (width 0.25) (layer F.Cu) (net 12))
 (segment (start 128.8701 76.3824) (end 126.8701 78.3824) (width 0.25) (layer F.Cu) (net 12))
 (segment (start 127.8201 82.3424) (end 129.3701 82.3424) (width 0.25) (layer F.Cu) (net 12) (status 20))
 (segment (start 126.8701 81.3924) (end 127.8201 82.3424) (width 0.25) (layer F.Cu) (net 12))
 (segment (start 151.3701 92.3824) (end 153.7501 92.3824) (width 0.25) (layer B.Cu) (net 5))
 (segment (start 153.7501 92.3824) (end 153.8301 92.4624) (width 0.25) (layer B.Cu) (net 5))
 (segment (start 146.5201 87.4224) (end 151.3701 92.2724) (width 0.25) (layer F.Cu) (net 5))
 (segment (start 151.3701 92.2724) (end 151.3701 92.3824) (width 0.25) (layer F.Cu) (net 5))
 (via (at 151.3701 92.3824) (size 0.6) (drill 0.3) (layers F.Cu B.Cu) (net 5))
 (segment (start 146.5201 87.4224) (end 146.0701 87.4224) (width 0.25) (layer F.Cu) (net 5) (status 30))
 (segment (start 153.8301 84.8424) (end 146.1101 84.8424) (width 0.25) (layer F.Cu) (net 1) (status 30))
 (segment (start 146.1101 84.8424) (end 146.0701 84.8824) (width 0.25) (layer F.Cu) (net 1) (status 30))
 (segment (start 146.5201 84.8824) (end 146.0701 84.8824) (width 0.25) (layer F.Cu) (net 1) (status 30))
 (segment (start 153.8601 82.3024) (end 146.1101 82.3024) (width 0.25) (layer F.Cu) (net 3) (status 30))
 (segment (start 146.1101 82.3024) (end 146.0701 82.3424) (width 0.25) (layer F.Cu) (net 3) (status 30))
 (segment (start 141.745101 81.697401) (end 141.1201 81.0724) (width 0.25) (layer F.Cu) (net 6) (status 20))
 (segment (start 141.745101 82.782407) (end 141.745101 81.697401) (width 0.25) (layer F.Cu) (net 6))
 (segment (start 141.1201 81.0724) (end 140.6701 81.0724) (width 0.25) (layer F.Cu) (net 6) (status 30))
 (segment (start 145.6201 86.1524) (end 145.0701 85.6024) (width 0.25) (layer F.Cu) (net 6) (status 10))
 (segment (start 146.0701 86.1524) (end 145.6201 86.1524) (width 0.25) (layer F.Cu) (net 6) (status 30))
 (segment (start 144.565094 85.6024) (end 141.745101 82.782407) (width 0.25) (layer F.Cu) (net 6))
 (segment (start 145.0701 85.6024) (end 144.565094 85.6024) (width 0.25) (layer F.Cu) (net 6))
 (segment (start 142.1001 86.1524) (end 142.847442 85.405058) (width 0.25) (layer F.Cu) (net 10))
 (segment (start 140.6701 86.1524) (end 142.1001 86.1524) (width 0.25) (layer F.Cu) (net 10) (status 10))
 (segment (start 146.0701 83.6124) (end 145.6201 83.6124) (width 0.25) (layer F.Cu) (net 10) (status 30))
 (segment (start 144.640104 83.6124) (end 144.070104 84.1824) (width 0.25) (layer F.Cu) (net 10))
 (segment (start 146.0701 83.6124) (end 144.640104 83.6124) (width 0.25) (layer F.Cu) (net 10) (status 10))
 (via (at 142.847442 85.405058) (size 0.6) (drill 0.3) (layers F.Cu B.Cu) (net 10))
 (via (at 144.070104 84.1824) (size 0.6) (drill 0.3) (layers F.Cu B.Cu) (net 10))
 (segment (start 144.0701 84.1824) (end 144.070104 84.1824) (width 0.25) (layer B.Cu) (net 10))
 (segment (start 142.847442 85.405058) (end 144.0701 84.1824) (width 0.25) (layer B.Cu) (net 10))
 (segment (start 140.6701 83.6124) (end 141.938683 83.6124) (width 0.25) (layer F.Cu) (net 8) (status 10))
 (segment (start 144.995099 86.668816) (end 144.995099 88.067399) (width 0.25) (layer F.Cu) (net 8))
 (segment (start 145.6201 88.6924) (end 146.0701 88.6924) (width 0.25) (layer F.Cu) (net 8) (status 30))
 (segment (start 144.995099 88.067399) (end 145.6201 88.6924) (width 0.25) (layer F.Cu) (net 8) (status 20))
 (segment (start 141.938683 83.6124) (end 144.995099 86.668816) (width 0.25) (layer F.Cu) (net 8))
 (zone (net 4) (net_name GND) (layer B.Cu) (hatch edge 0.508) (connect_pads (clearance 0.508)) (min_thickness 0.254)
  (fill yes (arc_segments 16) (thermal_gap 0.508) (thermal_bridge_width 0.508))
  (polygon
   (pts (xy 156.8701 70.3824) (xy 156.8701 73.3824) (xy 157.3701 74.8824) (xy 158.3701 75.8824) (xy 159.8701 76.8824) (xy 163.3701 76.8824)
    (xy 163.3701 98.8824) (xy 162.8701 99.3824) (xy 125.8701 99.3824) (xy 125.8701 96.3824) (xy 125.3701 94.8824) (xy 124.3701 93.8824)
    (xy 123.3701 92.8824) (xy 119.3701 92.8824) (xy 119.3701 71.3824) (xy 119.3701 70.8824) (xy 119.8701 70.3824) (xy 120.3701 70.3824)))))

